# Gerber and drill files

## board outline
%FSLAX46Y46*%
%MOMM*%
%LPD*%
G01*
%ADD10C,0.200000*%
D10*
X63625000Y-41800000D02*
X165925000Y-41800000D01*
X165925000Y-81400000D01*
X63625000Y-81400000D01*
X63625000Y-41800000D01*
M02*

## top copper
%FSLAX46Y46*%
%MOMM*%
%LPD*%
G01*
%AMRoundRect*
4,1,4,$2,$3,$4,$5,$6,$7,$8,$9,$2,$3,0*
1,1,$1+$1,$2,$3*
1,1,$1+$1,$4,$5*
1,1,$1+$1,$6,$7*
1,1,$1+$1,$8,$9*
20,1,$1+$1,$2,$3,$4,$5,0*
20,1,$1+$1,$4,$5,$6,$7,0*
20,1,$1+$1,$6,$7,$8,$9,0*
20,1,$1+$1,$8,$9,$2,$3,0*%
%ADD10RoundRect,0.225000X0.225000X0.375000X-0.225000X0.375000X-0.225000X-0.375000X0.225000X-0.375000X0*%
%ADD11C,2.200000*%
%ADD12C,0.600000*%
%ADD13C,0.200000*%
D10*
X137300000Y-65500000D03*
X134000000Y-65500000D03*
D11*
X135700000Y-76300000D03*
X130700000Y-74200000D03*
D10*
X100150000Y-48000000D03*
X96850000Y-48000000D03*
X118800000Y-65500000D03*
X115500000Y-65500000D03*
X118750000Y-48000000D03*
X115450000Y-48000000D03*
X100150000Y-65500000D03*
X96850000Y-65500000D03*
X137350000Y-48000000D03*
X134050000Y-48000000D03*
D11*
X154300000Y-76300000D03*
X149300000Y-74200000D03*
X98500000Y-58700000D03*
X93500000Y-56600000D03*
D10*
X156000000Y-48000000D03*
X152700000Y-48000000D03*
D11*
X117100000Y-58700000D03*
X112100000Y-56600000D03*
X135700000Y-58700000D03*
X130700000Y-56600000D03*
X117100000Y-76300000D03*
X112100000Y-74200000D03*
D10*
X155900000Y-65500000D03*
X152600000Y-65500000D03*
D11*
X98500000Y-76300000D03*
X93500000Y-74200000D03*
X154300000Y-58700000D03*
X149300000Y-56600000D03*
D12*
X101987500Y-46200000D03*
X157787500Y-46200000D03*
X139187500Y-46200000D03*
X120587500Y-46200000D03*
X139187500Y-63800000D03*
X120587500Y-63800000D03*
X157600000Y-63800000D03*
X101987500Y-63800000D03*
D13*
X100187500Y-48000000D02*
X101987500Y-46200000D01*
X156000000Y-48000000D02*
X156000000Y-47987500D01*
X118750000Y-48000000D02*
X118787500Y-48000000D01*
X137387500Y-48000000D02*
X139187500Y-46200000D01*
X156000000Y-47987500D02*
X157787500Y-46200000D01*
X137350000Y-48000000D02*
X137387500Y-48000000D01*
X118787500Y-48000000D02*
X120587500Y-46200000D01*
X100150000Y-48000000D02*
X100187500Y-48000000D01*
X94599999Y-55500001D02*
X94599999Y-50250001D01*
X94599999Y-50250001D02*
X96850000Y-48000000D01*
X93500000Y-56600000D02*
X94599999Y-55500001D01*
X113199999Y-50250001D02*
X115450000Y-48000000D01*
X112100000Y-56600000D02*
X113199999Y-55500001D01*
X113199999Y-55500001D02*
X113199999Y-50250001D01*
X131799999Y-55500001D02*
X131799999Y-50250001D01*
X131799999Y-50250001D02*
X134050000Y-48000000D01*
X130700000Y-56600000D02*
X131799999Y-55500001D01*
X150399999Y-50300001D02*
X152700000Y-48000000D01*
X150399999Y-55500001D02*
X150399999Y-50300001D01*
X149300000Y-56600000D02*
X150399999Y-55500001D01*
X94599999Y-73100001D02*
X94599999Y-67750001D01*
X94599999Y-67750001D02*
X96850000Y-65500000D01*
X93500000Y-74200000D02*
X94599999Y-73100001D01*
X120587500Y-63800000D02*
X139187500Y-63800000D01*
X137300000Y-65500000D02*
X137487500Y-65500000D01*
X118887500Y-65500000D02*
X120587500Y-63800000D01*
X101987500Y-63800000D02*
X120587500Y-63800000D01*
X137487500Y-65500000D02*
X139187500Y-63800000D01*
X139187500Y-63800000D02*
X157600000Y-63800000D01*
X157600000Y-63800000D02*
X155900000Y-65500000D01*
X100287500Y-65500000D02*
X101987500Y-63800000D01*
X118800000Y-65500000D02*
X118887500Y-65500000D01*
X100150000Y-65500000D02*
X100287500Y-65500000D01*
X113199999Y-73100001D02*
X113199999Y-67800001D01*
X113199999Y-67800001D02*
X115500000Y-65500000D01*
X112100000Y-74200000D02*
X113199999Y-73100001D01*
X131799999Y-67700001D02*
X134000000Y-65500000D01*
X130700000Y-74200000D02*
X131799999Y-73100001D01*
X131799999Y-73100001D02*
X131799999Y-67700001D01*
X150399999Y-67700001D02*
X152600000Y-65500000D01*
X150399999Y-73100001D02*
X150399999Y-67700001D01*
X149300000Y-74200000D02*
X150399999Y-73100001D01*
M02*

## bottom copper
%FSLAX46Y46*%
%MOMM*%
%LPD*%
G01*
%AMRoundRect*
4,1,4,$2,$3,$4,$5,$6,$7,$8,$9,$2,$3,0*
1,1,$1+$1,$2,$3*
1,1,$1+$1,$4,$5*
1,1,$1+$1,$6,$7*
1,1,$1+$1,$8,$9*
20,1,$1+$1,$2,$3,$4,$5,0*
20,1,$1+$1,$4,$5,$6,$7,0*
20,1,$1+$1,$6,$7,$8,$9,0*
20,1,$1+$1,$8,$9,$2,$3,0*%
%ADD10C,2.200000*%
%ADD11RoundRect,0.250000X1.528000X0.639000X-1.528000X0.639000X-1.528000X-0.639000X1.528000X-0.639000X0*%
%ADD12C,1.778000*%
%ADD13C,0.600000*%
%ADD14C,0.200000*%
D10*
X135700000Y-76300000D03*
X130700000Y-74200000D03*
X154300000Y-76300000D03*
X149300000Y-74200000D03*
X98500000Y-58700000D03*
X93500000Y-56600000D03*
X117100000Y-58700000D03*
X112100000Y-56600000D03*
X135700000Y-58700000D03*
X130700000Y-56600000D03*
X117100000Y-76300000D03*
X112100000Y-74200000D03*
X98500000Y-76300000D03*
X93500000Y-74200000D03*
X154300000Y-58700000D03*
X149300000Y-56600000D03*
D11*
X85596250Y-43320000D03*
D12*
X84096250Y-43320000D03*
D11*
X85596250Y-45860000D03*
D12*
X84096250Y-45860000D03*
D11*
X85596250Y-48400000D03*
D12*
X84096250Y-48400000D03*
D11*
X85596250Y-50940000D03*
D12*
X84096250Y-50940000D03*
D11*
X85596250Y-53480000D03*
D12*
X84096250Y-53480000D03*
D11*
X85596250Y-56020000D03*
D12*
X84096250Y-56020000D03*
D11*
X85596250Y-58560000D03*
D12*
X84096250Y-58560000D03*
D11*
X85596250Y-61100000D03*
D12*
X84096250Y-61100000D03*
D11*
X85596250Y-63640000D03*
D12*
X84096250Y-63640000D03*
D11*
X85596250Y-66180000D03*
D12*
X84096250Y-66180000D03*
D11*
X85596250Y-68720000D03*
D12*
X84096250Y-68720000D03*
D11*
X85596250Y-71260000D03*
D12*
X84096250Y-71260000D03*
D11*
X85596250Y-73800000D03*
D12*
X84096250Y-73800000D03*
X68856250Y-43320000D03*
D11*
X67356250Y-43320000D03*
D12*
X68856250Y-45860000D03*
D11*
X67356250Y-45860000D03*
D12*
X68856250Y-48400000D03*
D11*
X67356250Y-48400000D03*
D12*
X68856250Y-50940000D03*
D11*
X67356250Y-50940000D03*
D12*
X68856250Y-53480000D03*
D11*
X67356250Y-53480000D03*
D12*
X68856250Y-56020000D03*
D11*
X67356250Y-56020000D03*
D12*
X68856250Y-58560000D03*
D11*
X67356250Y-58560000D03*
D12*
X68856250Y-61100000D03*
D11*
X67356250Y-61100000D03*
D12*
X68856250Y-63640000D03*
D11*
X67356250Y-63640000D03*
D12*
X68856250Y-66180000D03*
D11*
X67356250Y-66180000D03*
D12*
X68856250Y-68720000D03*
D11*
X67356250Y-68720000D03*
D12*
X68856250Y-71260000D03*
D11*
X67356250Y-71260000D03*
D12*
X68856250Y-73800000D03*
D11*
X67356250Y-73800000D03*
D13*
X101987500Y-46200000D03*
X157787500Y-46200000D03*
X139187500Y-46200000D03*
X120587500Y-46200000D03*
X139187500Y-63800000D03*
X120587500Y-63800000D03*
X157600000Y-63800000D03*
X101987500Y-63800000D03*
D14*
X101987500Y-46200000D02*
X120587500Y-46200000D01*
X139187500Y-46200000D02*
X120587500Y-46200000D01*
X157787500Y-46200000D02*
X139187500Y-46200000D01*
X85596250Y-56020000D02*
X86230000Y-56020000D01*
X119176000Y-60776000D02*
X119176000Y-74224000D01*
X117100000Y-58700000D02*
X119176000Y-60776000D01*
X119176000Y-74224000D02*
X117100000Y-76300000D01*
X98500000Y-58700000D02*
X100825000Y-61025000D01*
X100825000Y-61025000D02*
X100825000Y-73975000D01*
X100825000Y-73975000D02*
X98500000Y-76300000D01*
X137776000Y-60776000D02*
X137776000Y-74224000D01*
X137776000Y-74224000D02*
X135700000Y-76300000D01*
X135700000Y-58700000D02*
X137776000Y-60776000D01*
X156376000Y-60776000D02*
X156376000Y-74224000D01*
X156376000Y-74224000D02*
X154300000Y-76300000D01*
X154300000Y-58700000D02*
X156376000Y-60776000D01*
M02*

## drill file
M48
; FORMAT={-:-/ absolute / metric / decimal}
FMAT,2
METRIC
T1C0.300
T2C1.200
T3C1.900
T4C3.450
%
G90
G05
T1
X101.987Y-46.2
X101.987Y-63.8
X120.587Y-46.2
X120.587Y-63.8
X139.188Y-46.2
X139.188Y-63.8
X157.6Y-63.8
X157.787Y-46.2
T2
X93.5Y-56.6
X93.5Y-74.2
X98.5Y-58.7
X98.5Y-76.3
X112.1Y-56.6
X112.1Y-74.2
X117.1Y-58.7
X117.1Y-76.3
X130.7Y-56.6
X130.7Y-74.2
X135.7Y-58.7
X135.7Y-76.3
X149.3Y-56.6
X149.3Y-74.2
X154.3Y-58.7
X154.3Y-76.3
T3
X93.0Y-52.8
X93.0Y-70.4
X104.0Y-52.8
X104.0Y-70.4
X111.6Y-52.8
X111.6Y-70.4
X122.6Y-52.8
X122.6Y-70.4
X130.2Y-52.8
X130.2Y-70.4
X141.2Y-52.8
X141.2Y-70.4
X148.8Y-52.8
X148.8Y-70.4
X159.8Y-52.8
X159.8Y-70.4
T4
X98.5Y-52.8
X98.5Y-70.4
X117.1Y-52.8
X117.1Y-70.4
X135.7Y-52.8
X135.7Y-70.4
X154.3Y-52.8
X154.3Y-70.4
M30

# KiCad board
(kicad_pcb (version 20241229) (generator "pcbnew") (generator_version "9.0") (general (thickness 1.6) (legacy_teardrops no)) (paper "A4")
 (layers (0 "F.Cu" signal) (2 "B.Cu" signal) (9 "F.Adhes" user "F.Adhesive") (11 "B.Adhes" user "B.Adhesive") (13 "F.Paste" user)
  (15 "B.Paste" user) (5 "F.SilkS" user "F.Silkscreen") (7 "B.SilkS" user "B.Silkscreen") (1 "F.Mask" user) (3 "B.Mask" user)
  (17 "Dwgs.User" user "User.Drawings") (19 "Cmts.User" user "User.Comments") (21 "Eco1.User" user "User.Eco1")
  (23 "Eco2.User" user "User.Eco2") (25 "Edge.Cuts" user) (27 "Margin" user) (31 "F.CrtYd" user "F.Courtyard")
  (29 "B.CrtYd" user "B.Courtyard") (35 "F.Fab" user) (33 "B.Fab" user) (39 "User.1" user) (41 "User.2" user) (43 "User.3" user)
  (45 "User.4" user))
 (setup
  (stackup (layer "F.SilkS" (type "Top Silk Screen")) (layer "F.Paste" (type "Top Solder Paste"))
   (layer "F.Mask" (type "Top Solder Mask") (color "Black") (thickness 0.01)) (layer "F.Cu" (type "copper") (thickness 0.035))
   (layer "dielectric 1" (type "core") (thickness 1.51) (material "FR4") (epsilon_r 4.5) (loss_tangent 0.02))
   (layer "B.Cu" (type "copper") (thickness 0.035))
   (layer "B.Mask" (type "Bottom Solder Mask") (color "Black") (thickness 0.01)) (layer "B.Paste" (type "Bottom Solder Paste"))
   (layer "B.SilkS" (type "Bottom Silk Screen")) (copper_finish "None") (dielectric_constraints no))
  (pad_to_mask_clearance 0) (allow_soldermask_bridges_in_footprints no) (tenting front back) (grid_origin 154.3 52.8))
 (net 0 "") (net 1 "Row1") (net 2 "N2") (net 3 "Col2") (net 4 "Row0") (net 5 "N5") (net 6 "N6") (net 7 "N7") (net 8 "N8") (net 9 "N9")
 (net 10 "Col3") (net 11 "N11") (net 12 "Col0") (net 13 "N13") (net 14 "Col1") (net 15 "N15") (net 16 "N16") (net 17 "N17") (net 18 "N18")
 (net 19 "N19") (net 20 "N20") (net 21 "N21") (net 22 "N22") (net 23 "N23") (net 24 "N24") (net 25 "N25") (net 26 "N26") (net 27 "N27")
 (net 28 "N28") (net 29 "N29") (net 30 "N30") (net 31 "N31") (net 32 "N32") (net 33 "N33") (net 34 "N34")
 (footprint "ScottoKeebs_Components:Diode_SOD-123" (layer "F.Cu") (at 135.65 65.5 180)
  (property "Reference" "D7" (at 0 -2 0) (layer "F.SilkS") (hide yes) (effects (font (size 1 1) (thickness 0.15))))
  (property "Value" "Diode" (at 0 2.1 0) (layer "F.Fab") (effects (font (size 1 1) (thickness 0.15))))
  (pad "1" smd roundrect (at -1.65 0 180) (size 0.9 1.2) (layers "F.Cu" "F.Mask" "F.Paste") (roundrect_rratio 0.25) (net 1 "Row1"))
  (pad "2" smd roundrect (at 1.65 0 180) (size 0.9 1.2) (layers "F.Cu" "F.Mask" "F.Paste") (roundrect_rratio 0.25) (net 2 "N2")))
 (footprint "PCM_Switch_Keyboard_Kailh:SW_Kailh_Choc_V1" (layer "F.Cu") (at 135.7 70.4 180)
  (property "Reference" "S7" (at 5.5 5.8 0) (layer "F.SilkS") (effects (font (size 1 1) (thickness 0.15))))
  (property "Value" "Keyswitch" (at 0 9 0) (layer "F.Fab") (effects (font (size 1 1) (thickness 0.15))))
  (pad "" np_thru_hole circle (at -5.5 0 180) (size 1.9 1.9) (drill 1.9) (layers "*.Cu" "*.Mask"))
  (pad "" np_thru_hole circle (at 0 0 180) (size 3.45 3.45) (drill 3.45) (layers "*.Cu" "*.Mask"))
  (pad "" np_thru_hole circle (at 5.5 0 180) (size 1.9 1.9) (drill 1.9) (layers "*.Cu" "*.Mask"))
  (pad "1" thru_hole circle (at 0 -5.9 180) (size 2.2 2.2) (drill 1.2) (layers "*.Cu" "*.Mask") (remove_unused_layers no) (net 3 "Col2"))
  (pad "2" thru_hole circle (at 5 -3.8 180) (size 2.2 2.2) (drill 1.2) (layers "*.Cu" "*.Mask") (remove_unused_layers no) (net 2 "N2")))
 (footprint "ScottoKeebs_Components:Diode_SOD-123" (layer "F.Cu") (at 98.5 48 180)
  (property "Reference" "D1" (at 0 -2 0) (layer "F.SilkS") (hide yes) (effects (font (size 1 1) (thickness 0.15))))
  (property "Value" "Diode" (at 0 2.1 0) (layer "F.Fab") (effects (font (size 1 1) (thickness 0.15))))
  (pad "1" smd roundrect (at -1.65 0 180) (size 0.9 1.2) (layers "F.Cu" "F.Mask" "F.Paste") (roundrect_rratio 0.25) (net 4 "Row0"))
  (pad "2" smd roundrect (at 1.65 0 180) (size 0.9 1.2) (layers "F.Cu" "F.Mask" "F.Paste") (roundrect_rratio 0.25) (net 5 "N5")))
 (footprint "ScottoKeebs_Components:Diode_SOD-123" (layer "F.Cu") (at 117.15 65.5 180)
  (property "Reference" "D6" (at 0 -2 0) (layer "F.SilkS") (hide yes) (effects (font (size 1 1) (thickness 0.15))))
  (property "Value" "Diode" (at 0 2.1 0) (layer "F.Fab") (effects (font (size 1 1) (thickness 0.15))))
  (pad "1" smd roundrect (at -1.65 0 180) (size 0.9 1.2) (layers "F.Cu" "F.Mask" "F.Paste") (roundrect_rratio 0.25) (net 1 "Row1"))
  (pad "2" smd roundrect (at 1.65 0 180) (size 0.9 1.2) (layers "F.Cu" "F.Mask" "F.Paste") (roundrect_rratio 0.25) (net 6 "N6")))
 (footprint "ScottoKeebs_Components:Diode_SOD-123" (layer "F.Cu") (at 117.1 48 180)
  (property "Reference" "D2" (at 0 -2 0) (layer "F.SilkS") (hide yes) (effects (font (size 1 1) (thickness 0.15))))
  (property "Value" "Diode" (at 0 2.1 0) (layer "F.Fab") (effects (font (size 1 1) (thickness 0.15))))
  (pad "1" smd roundrect (at -1.65 0 180) (size 0.9 1.2) (layers "F.Cu" "F.Mask" "F.Paste") (roundrect_rratio 0.25) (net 4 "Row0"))
  (pad "2" smd roundrect (at 1.65 0 180) (size 0.9 1.2) (layers "F.Cu" "F.Mask" "F.Paste") (roundrect_rratio 0.25) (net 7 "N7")))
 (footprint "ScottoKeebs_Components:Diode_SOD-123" (layer "F.Cu") (at 98.5 65.5 180)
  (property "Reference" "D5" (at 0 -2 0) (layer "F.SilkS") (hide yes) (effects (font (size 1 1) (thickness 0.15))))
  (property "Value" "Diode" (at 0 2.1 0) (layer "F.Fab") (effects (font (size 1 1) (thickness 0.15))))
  (pad "1" smd roundrect (at -1.65 0 180) (size 0.9 1.2) (layers "F.Cu" "F.Mask" "F.Paste") (roundrect_rratio 0.25) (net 1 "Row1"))
  (pad "2" smd roundrect (at 1.65 0 180) (size 0.9 1.2) (layers "F.Cu" "F.Mask" "F.Paste") (roundrect_rratio 0.25) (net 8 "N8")))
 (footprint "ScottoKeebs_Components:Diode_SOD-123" (layer "F.Cu") (at 135.7 48 180)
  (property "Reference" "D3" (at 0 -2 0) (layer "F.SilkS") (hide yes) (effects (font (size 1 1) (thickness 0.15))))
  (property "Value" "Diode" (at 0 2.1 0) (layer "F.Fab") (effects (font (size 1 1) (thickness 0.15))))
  (pad "1" smd roundrect (at -1.65 0 180) (size 0.9 1.2) (layers "F.Cu" "F.Mask" "F.Paste") (roundrect_rratio 0.25) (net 4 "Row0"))
  (pad "2" smd roundrect (at 1.65 0 180) (size 0.9 1.2) (layers "F.Cu" "F.Mask" "F.Paste") (roundrect_rratio 0.25) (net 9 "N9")))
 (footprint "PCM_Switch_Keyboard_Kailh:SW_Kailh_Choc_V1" (layer "F.Cu") (at 154.3 70.4 180)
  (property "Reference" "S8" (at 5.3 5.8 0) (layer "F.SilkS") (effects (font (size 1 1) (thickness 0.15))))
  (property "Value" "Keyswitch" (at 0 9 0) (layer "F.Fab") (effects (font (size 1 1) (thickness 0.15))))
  (pad "" np_thru_hole circle (at -5.5 0 180) (size 1.9 1.9) (drill 1.9) (layers "*.Cu" "*.Mask"))
  (pad "" np_thru_hole circle (at 0 0 180) (size 3.45 3.45) (drill 3.45) (layers "*.Cu" "*.Mask"))
  (pad "" np_thru_hole circle (at 5.5 0 180) (size 1.9 1.9) (drill 1.9) (layers "*.Cu" "*.Mask"))
  (pad "1" thru_hole circle (at 0 -5.9 180) (size 2.2 2.2) (drill 1.2) (layers "*.Cu" "*.Mask") (remove_unused_layers no) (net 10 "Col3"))
  (pad "2" thru_hole circle (at 5 -3.8 180) (size 2.2 2.2) (drill 1.2) (layers "*.Cu" "*.Mask") (remove_unused_layers no) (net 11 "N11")))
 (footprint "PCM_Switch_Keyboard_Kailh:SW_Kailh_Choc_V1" (layer "F.Cu") (at 98.5 52.8 180)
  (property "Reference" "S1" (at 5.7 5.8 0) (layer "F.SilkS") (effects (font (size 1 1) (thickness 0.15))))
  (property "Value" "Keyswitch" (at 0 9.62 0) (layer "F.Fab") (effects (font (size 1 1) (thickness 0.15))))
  (pad "" np_thru_hole circle (at -5.5 0 180) (size 1.9 1.9) (drill 1.9) (layers "*.Cu" "*.Mask"))
  (pad "" np_thru_hole circle (at 0 0 180) (size 3.45 3.45) (drill 3.45) (layers "*.Cu" "*.Mask"))
  (pad "" np_thru_hole circle (at 5.5 0 180) (size 1.9 1.9) (drill 1.9) (layers "*.Cu" "*.Mask"))
  (pad "1" thru_hole circle (at 0 -5.9 180) (size 2.2 2.2) (drill 1.2) (layers "*.Cu" "*.Mask") (remove_unused_layers no) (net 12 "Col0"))
  (pad "2" thru_hole circle (at 5 -3.8 180) (size 2.2 2.2) (drill 1.2) (layers "*.Cu" "*.Mask") (remove_unused_layers no) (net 5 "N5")))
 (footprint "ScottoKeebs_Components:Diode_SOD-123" (layer "F.Cu") (at 154.35 48 180)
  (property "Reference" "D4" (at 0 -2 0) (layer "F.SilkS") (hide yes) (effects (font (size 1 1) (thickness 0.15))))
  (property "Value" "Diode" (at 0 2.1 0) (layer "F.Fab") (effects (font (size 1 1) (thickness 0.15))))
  (pad "1" smd roundrect (at -1.65 0 180) (size 0.9 1.2) (layers "F.Cu" "F.Mask" "F.Paste") (roundrect_rratio 0.25) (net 4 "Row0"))
  (pad "2" smd roundrect (at 1.65 0 180) (size 0.9 1.2) (layers "F.Cu" "F.Mask" "F.Paste") (roundrect_rratio 0.25) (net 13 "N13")))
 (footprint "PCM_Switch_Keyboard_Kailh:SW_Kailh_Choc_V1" (layer "F.Cu") (at 117.1 52.8 180)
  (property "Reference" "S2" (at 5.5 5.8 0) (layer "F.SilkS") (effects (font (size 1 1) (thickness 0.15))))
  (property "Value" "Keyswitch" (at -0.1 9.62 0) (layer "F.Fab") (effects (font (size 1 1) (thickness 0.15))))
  (pad "" np_thru_hole circle (at -5.5 0 180) (size 1.9 1.9) (drill 1.9) (layers "*.Cu" "*.Mask"))
  (pad "" np_thru_hole circle (at 0 0 180) (size 3.45 3.45) (drill 3.45) (layers "*.Cu" "*.Mask"))
  (pad "" np_thru_hole circle (at 5.5 0 180) (size 1.9 1.9) (drill 1.9) (layers "*.Cu" "*.Mask"))
  (pad "1" thru_hole circle (at 0 -5.9 180) (size 2.2 2.2) (drill 1.2) (layers "*.Cu" "*.Mask") (remove_unused_layers no) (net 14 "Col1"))
  (pad "2" thru_hole circle (at 5 -3.8 180) (size 2.2 2.2) (drill 1.2) (layers "*.Cu" "*.Mask") (remove_unused_layers no) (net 7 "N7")))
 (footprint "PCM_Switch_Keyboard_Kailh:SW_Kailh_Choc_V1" (layer "F.Cu") (at 135.7 52.8 180)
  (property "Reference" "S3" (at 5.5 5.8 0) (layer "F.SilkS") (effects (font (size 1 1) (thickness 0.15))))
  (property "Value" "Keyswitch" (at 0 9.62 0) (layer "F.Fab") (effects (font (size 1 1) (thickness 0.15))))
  (pad "" np_thru_hole circle (at -5.5 0 180) (size 1.9 1.9) (drill 1.9) (layers "*.Cu" "*.Mask"))
  (pad "" np_thru_hole circle (at 0 0 180) (size 3.45 3.45) (drill 3.45) (layers "*.Cu" "*.Mask"))
  (pad "" np_thru_hole circle (at 5.5 0 180) (size 1.9 1.9) (drill 1.9) (layers "*.Cu" "*.Mask"))
  (pad "1" thru_hole circle (at 0 -5.9 180) (size 2.2 2.2) (drill 1.2) (layers "*.Cu" "*.Mask") (remove_unused_layers no) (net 3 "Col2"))
  (pad "2" thru_hole circle (at 5 -3.8 180) (size 2.2 2.2) (drill 1.2) (layers "*.Cu" "*.Mask") (remove_unused_layers no) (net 9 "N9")))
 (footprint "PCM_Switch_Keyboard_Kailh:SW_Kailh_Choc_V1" (layer "F.Cu") (at 117.1 70.4 180)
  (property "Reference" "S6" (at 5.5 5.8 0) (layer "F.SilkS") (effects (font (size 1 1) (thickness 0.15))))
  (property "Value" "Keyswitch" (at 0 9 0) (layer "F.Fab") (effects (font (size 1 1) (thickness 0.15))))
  (pad "" np_thru_hole circle (at -5.5 0 180) (size 1.9 1.9) (drill 1.9) (layers "*.Cu" "*.Mask"))
  (pad "" np_thru_hole circle (at 0 0 180) (size 3.45 3.45) (drill 3.45) (layers "*.Cu" "*.Mask"))
  (pad "" np_thru_hole circle (at 5.5 0 180) (size 1.9 1.9) (drill 1.9) (layers "*.Cu" "*.Mask"))
  (pad "1" thru_hole circle (at 0 -5.9 180) (size 2.2 2.2) (drill 1.2) (layers "*.Cu" "*.Mask") (remove_unused_layers no) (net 14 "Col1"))
  (pad "2" thru_hole circle (at 5 -3.8 180) (size 2.2 2.2) (drill 1.2) (layers "*.Cu" "*.Mask") (remove_unused_layers no) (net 6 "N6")))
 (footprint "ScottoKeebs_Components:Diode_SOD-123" (layer "F.Cu") (at 154.25 65.5 180)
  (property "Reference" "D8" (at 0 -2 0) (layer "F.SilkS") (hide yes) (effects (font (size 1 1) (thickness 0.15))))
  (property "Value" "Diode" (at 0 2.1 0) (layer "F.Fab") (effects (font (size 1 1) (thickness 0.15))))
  (pad "1" smd roundrect (at -1.65 0 180) (size 0.9 1.2) (layers "F.Cu" "F.Mask" "F.Paste") (roundrect_rratio 0.25) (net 1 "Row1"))
  (pad "2" smd roundrect (at 1.65 0 180) (size 0.9 1.2) (layers "F.Cu" "F.Mask" "F.Paste") (roundrect_rratio 0.25) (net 11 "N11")))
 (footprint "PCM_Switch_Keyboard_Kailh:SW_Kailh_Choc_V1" (layer "F.Cu") (at 98.5 70.4 180)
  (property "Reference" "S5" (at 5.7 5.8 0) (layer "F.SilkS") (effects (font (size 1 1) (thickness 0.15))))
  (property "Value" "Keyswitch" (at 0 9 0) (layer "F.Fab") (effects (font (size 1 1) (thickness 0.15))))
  (pad "" np_thru_hole circle (at -5.5 0 180) (size 1.9 1.9) (drill 1.9) (layers "*.Cu" "*.Mask"))
  (pad "" np_thru_hole circle (at 0 0 180) (size 3.45 3.45) (drill 3.45) (layers "*.Cu" "*.Mask"))
  (pad "" np_thru_hole circle (at 5.5 0 180) (size 1.9 1.9) (drill 1.9) (layers "*.Cu" "*.Mask"))
  (pad "1" thru_hole circle (at 0 -5.9 180) (size 2.2 2.2) (drill 1.2) (layers "*.Cu" "*.Mask") (remove_unused_layers no) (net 12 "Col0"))
  (pad "2" thru_hole circle (at 5 -3.8 180) (size 2.2 2.2) (drill 1.2) (layers "*.Cu" "*.Mask") (remove_unused_layers no) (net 8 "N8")))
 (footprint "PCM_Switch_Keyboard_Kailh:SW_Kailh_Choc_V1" (layer "F.Cu") (at 154.3 52.8 180)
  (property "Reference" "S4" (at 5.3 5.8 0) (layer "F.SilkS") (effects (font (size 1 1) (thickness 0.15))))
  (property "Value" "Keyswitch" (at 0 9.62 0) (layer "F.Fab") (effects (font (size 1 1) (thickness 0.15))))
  (pad "" np_thru_hole circle (at -5.5 0 180) (size 1.9 1.9) (drill 1.9) (layers "*.Cu" "*.Mask"))
  (pad "" np_thru_hole circle (at 0 0 180) (size 3.45 3.45) (drill 3.45) (layers "*.Cu" "*.Mask"))
  (pad "" np_thru_hole circle (at 5.5 0 180) (size 1.9 1.9) (drill 1.9) (layers "*.Cu" "*.Mask"))
  (pad "1" thru_hole circle (at 0 -5.9 180) (size 2.2 2.2) (drill 1.2) (layers "*.Cu" "*.Mask") (remove_unused_layers no) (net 10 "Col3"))
  (pad "2" thru_hole circle (at 5 -3.8 180) (size 2.2 2.2) (drill 1.2) (layers "*.Cu" "*.Mask") (remove_unused_layers no) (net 13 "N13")))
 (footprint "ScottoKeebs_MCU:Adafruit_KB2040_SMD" (layer "B.Cu") (at 76.48625 58.55 180)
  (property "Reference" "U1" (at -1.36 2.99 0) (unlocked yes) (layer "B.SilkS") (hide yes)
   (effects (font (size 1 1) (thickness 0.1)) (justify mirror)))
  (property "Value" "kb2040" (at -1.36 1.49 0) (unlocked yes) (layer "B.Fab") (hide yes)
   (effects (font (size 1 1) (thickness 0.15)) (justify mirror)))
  (pad "1" smd roundrect (at -9.11 15.23 180) (size 3.556 1.778) (layers "B.Cu" "B.Mask") (roundrect_rratio 0.1406074241) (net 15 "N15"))
  (pad "1" smd circle (at -7.61 15.23 180) (size 1.778 1.778) (layers "B.Cu" "B.Mask" "B.Paste") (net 15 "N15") (solder_mask_margin 0.0508)
   (thermal_bridge_angle 0))
  (pad "2" smd roundrect (at -9.11 12.69 180) (size 3.556 1.778) (layers "B.Cu" "B.Mask") (roundrect_rratio 0.1406074241) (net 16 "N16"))
  (pad "2" smd circle (at -7.61 12.69 180) (size 1.778 1.778) (layers "B.Cu" "B.Mask" "B.Paste") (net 16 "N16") (solder_mask_margin 0.0508)
   (thermal_bridge_angle 0))
  (pad "3" smd roundrect (at -9.11 10.15 180) (size 3.556 1.778) (layers "B.Cu" "B.Mask") (roundrect_rratio 0.1406074241) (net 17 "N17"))
  (pad "3" smd circle (at -7.61 10.15 180) (size 1.778 1.778) (layers "B.Cu" "B.Mask" "B.Paste") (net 17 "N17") (solder_mask_margin 0.0508)
   (thermal_bridge_angle 0))
  (pad "4" smd roundrect (at -9.11 7.61 180) (size 3.556 1.778) (layers "B.Cu" "B.Mask") (roundrect_rratio 0.1406074241) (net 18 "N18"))
  (pad "4" smd circle (at -7.61 7.61 180) (size 1.778 1.778) (layers "B.Cu" "B.Mask" "B.Paste") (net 18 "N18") (solder_mask_margin 0.0508)
   (thermal_bridge_angle 0))
  (pad "5" smd roundrect (at -9.11 5.07 180) (size 3.556 1.778) (layers "B.Cu" "B.Mask") (roundrect_rratio 0.1406074241) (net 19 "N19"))
  (pad "5" smd circle (at -7.61 5.07 180) (size 1.778 1.778) (layers "B.Cu" "B.Mask" "B.Paste") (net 19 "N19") (solder_mask_margin 0.0508)
   (thermal_bridge_angle 0))
  (pad "6" smd roundrect (at -9.11 2.53 180) (size 3.556 1.778) (layers "B.Cu" "B.Mask") (roundrect_rratio 0.1406074241) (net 1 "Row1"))
  (pad "6" smd circle (at -7.61 2.53 180) (size 1.778 1.778) (layers "B.Cu" "B.Mask" "B.Paste") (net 1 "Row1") (solder_mask_margin 0.0508)
   (thermal_bridge_angle 0))
  (pad "7" smd roundrect (at -9.11 -0.01 180) (size 3.556 1.778) (layers "B.Cu" "B.Mask") (roundrect_rratio 0.1406074241) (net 4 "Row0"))
  (pad "7" smd circle (at -7.61 -0.01 180) (size 1.778 1.778) (layers "B.Cu" "B.Mask" "B.Paste") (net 4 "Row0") (solder_mask_margin 0.0508)
   (thermal_bridge_angle 0))
  (pad "8" smd roundrect (at -9.11 -2.55 180) (size 3.556 1.778) (layers "B.Cu" "B.Mask") (roundrect_rratio 0.1406074241) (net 10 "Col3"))
  (pad "8" smd circle (at -7.61 -2.55 180) (size 1.778 1.778) (layers "B.Cu" "B.Mask" "B.Paste") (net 10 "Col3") (solder_mask_margin 0.0508)
   (thermal_bridge_angle 0))
  (pad "9" smd roundrect (at -9.11 -5.09 180) (size 3.556 1.778) (layers "B.Cu" "B.Mask") (roundrect_rratio 0.1406074241) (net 3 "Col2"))
  (pad "9" smd circle (at -7.61 -5.09 180) (size 1.778 1.778) (layers "B.Cu" "B.Mask" "B.Paste") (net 3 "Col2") (solder_mask_margin 0.0508)
   (thermal_bridge_angle 0))
  (pad "10" smd roundrect (at -9.11 -7.63 180) (size 3.556 1.778) (layers "B.Cu" "B.Mask") (roundrect_rratio 0.1406074241) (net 14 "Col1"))
  (pad "10" smd circle (at -7.61 -7.63 180) (size 1.778 1.778) (layers "B.Cu" "B.Mask" "B.Paste") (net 14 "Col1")
   (solder_mask_margin 0.0508) (thermal_bridge_angle 0))
  (pad "11" smd roundrect (at -9.11 -10.17 180) (size 3.556 1.778) (layers "B.Cu" "B.Mask") (roundrect_rratio 0.1406074241) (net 12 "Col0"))
  (pad "11" smd circle (at -7.61 -10.17 180) (size 1.778 1.778) (layers "B.Cu" "B.Mask" "B.Paste") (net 12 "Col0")
   (solder_mask_margin 0.0508) (thermal_bridge_angle 0))
  (pad "12" smd roundrect (at -9.11 -12.71 180) (size 3.556 1.778) (layers "B.Cu" "B.Mask") (roundrect_rratio 0.1406074241) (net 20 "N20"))
  (pad "12" smd circle (at -7.61 -12.71 180) (size 1.778 1.778) (layers "B.Cu" "B.Mask" "B.Paste") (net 20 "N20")
   (solder_mask_margin 0.0508) (thermal_bridge_angle 0))
  (pad "13" smd roundrect (at -9.11 -15.25 180) (size 3.556 1.778) (layers "B.Cu" "B.Mask") (roundrect_rratio 0.1406074241) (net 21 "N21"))
  (pad "13" smd circle (at -7.61 -15.25 180) (size 1.778 1.778) (layers "B.Cu" "B.Mask" "B.Paste") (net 21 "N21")
   (solder_mask_margin 0.0508) (thermal_bridge_angle 0))
  (pad "14" smd circle (at 7.63 15.23 180) (size 1.778 1.778) (layers "B.Cu" "B.Mask" "B.Paste") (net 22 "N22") (solder_mask_margin 0.0508)
   (thermal_bridge_angle 0))
  (pad "14" smd roundrect (at 9.13 15.23 180) (size 3.556 1.778) (layers "B.Cu" "B.Mask") (roundrect_rratio 0.1406074241) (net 22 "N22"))
  (pad "15" smd circle (at 7.63 12.69 180) (size 1.778 1.778) (layers "B.Cu" "B.Mask" "B.Paste") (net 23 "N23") (solder_mask_margin 0.0508)
   (thermal_bridge_angle 0))
  (pad "15" smd roundrect (at 9.13 12.69 180) (size 3.556 1.778) (layers "B.Cu" "B.Mask") (roundrect_rratio 0.1406074241) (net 23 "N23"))
  (pad "16" smd circle (at 7.63 10.15 180) (size 1.778 1.778) (layers "B.Cu" "B.Mask" "B.Paste") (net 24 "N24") (solder_mask_margin 0.0508)
   (thermal_bridge_angle 0))
  (pad "16" smd roundrect (at 9.13 10.15 180) (size 3.556 1.778) (layers "B.Cu" "B.Mask") (roundrect_rratio 0.1406074241) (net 24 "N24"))
  (pad "17" smd circle (at 7.63 7.61 180) (size 1.778 1.778) (layers "B.Cu" "B.Mask" "B.Paste") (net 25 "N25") (solder_mask_margin 0.0508)
   (thermal_bridge_angle 0))
  (pad "17" smd roundrect (at 9.13 7.61 180) (size 3.556 1.778) (layers "B.Cu" "B.Mask") (roundrect_rratio 0.1406074241) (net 25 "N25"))
  (pad "18" smd circle (at 7.63 5.07 180) (size 1.778 1.778) (layers "B.Cu" "B.Mask" "B.Paste") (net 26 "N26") (solder_mask_margin 0.0508)
   (thermal_bridge_angle 0))
  (pad "18" smd roundrect (at 9.13 5.07 180) (size 3.556 1.778) (layers "B.Cu" "B.Mask") (roundrect_rratio 0.1406074241) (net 26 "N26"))
  (pad "19" smd circle (at 7.63 2.53 180) (size 1.778 1.778) (layers "B.Cu" "B.Mask" "B.Paste") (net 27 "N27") (solder_mask_margin 0.0508)
   (thermal_bridge_angle 0))
  (pad "19" smd roundrect (at 9.13 2.53 180) (size 3.556 1.778) (layers "B.Cu" "B.Mask") (roundrect_rratio 0.1406074241) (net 27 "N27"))
  (pad "20" smd circle (at 7.63 -0.01 180) (size 1.778 1.778) (layers "B.Cu" "B.Mask" "B.Paste") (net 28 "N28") (solder_mask_margin 0.0508)
   (thermal_bridge_angle 0))
  (pad "20" smd roundrect (at 9.13 -0.01 180) (size 3.556 1.778) (layers "B.Cu" "B.Mask") (roundrect_rratio 0.1406074241) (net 28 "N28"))
  (pad "21" smd circle (at 7.63 -2.55 180) (size 1.778 1.778) (layers "B.Cu" "B.Mask" "B.Paste") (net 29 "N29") (solder_mask_margin 0.0508)
   (thermal_bridge_angle 0))
  (pad "21" smd roundrect (at 9.13 -2.55 180) (size 3.556 1.778) (layers "B.Cu" "B.Mask") (roundrect_rratio 0.1406074241) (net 29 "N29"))
  (pad "22" smd circle (at 7.63 -5.09 180) (size 1.778 1.778) (layers "B.Cu" "B.Mask" "B.Paste") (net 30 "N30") (solder_mask_margin 0.0508)
   (thermal_bridge_angle 0))
  (pad "22" smd roundrect (at 9.13 -5.09 180) (size 3.556 1.778) (layers "B.Cu" "B.Mask") (roundrect_rratio 0.1406074241) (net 30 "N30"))
  (pad "23" smd circle (at 7.63 -7.63 180) (size 1.778 1.778) (layers "B.Cu" "B.Mask" "B.Paste") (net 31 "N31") (solder_mask_margin 0.0508)
   (thermal_bridge_angle 0))
  (pad "23" smd roundrect (at 9.13 -7.63 180) (size 3.556 1.778) (layers "B.Cu" "B.Mask") (roundrect_rratio 0.1406074241) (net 31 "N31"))
  (pad "24" smd circle (at 7.63 -10.17 180) (size 1.778 1.778) (layers "B.Cu" "B.Mask" "B.Paste") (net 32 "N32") (solder_mask_margin 0.0508)
   (thermal_bridge_angle 0))
  (pad "24" smd roundrect (at 9.13 -10.17 180) (size 3.556 1.778) (layers "B.Cu" "B.Mask") (roundrect_rratio 0.1406074241) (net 32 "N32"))
  (pad "25" smd circle (at 7.63 -12.71 180) (size 1.778 1.778) (layers "B.Cu" "B.Mask" "B.Paste") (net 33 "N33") (solder_mask_margin 0.0508)
   (thermal_bridge_angle 0))
  (pad "25" smd roundrect (at 9.13 -12.71 180) (size 3.556 1.778) (layers "B.Cu" "B.Mask") (roundrect_rratio 0.1406074241) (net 33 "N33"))
  (pad "26" smd circle (at 7.63 -15.25 180) (size 1.778 1.778) (layers "B.Cu" "B.Mask" "B.Paste") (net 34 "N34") (solder_mask_margin 0.0508)
   (thermal_bridge_angle 0))
  (pad "26" smd roundrect (at 9.13 -15.25 180) (size 3.556 1.778) (layers "B.Cu" "B.Mask") (roundrect_rratio 0.1406074241) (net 34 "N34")))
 (gr_rect (start 63.625 41.8) (end 165.925 81.4) (stroke (width 0.2) (type solid)) (fill no) (layer "Edge.Cuts"))
 (segment (start 100.1875 48) (end 101.9875 46.2) (width 0.2) (layer "F.Cu") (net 4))
 (segment (start 156 48) (end 156 47.9875) (width 0.2) (layer "F.Cu") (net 4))
 (segment (start 118.75 48) (end 118.7875 48) (width 0.2) (layer "F.Cu") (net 4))
 (segment (start 137.3875 48) (end 139.1875 46.2) (width 0.2) (layer "F.Cu") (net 4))
 (segment (start 156 47.9875) (end 157.7875 46.2) (width 0.2) (layer "F.Cu") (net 4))
 (segment (start 137.35 48) (end 137.3875 48) (width 0.2) (layer "F.Cu") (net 4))
 (segment (start 118.7875 48) (end 120.5875 46.2) (width 0.2) (layer "F.Cu") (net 4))
 (segment (start 100.15 48) (end 100.1875 48) (width 0.2) (layer "F.Cu") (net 4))
 (via (at 101.9875 46.2) (size 0.6) (drill 0.3) (layers "F.Cu" "B.Cu") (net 4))
 (via (at 157.7875 46.2) (size 0.6) (drill 0.3) (layers "F.Cu" "B.Cu") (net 4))
 (via (at 139.1875 46.2) (size 0.6) (drill 0.3) (layers "F.Cu" "B.Cu") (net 4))
 (via (at 120.5875 46.2) (size 0.6) (drill 0.3) (layers "F.Cu" "B.Cu") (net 4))
 (segment (start 101.9875 46.2) (end 120.5875 46.2) (width 0.2) (layer "B.Cu") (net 4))
 (segment (start 139.1875 46.2) (end 120.5875 46.2) (width 0.2) (layer "B.Cu") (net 4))
 (segment (start 157.7875 46.2) (end 139.1875 46.2) (width 0.2) (layer "B.Cu") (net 4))
 (segment (start 94.599999 55.500001) (end 94.599999 50.250001) (width 0.2) (layer "F.Cu") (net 5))
 (segment (start 94.599999 50.250001) (end 96.85 48) (width 0.2) (layer "F.Cu") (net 5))
 (segment (start 93.5 56.6) (end 94.599999 55.500001) (width 0.2) (layer "F.Cu") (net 5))
 (segment (start 113.199999 50.250001) (end 115.45 48) (width 0.2) (layer "F.Cu") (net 7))
 (segment (start 112.1 56.6) (end 113.199999 55.500001) (width 0.2) (layer "F.Cu") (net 7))
 (segment (start 113.199999 55.500001) (end 113.199999 50.250001) (width 0.2) (layer "F.Cu") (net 7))
 (segment (start 131.799999 55.500001) (end 131.799999 50.250001) (width 0.2) (layer "F.Cu") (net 9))
 (segment (start 131.799999 50.250001) (end 134.05 48) (width 0.2) (layer "F.Cu") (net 9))
 (segment (start 130.7 56.6) (end 131.799999 55.500001) (width 0.2) (layer "F.Cu") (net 9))
 (segment (start 150.399999 50.300001) (end 152.7 48) (width 0.2) (layer "F.Cu") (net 13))
 (segment (start 150.399999 55.500001) (end 150.399999 50.300001) (width 0.2) (layer "F.Cu") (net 13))
 (segment (start 149.3 56.6) (end 150.399999 55.500001) (width 0.2) (layer "F.Cu") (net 13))
 (segment (start 94.599999 73.100001) (end 94.599999 67.750001) (width 0.2) (layer "F.Cu") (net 8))
 (segment (start 94.599999 67.750001) (end 96.85 65.5) (width 0.2) (layer "F.Cu") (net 8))
 (segment (start 93.5 74.2) (end 94.599999 73.100001) (width 0.2) (layer "F.Cu") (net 8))
 (segment (start 120.5875 63.8) (end 139.1875 63.8) (width 0.2) (layer "F.Cu") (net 1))
 (segment (start 137.3 65.5) (end 137.4875 65.5) (width 0.2) (layer "F.Cu") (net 1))
 (segment (start 118.8875 65.5) (end 120.5875 63.8) (width 0.2) (layer "F.Cu") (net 1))
 (segment (start 101.9875 63.8) (end 120.5875 63.8) (width 0.2) (layer "F.Cu") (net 1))
 (segment (start 137.4875 65.5) (end 139.1875 63.8) (width 0.2) (layer "F.Cu") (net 1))
 (segment (start 139.1875 63.8) (end 157.6 63.8) (width 0.2) (layer "F.Cu") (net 1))
 (segment (start 157.6 63.8) (end 155.9 65.5) (width 0.2) (layer "F.Cu") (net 1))
 (segment (start 100.2875 65.5) (end 101.9875 63.8) (width 0.2) (layer "F.Cu") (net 1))
 (segment (start 118.8 65.5) (end 118.8875 65.5) (width 0.2) (layer "F.Cu") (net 1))
 (segment (start 100.15 65.5) (end 100.2875 65.5) (width 0.2) (layer "F.Cu") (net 1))
 (via (at 139.1875 63.8) (size 0.6) (drill 0.3) (layers "F.Cu" "B.Cu") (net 1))
 (via (at 120.5875 63.8) (size 0.6) (drill 0.3) (layers "F.Cu" "B.Cu") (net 1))
 (via (at 157.6 63.8) (size 0.6) (drill 0.3) (layers "F.Cu" "B.Cu") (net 1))
 (via (at 101.9875 63.8) (size 0.6) (drill 0.3) (layers "F.Cu" "B.Cu") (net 1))
 (segment (start 85.59625 56.02) (end 86.23 56.02) (width 0.2) (layer "B.Cu") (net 1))
 (segment (start 113.199999 73.100001) (end 113.199999 67.800001) (width 0.2) (layer "F.Cu") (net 6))
 (segment (start 113.199999 67.800001) (end 115.5 65.5) (width 0.2) (layer "F.Cu") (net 6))
 (segment (start 112.1 74.2) (end 113.199999 73.100001) (width 0.2) (layer "F.Cu") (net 6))
 (segment (start 131.799999 67.700001) (end 134 65.5) (width 0.2) (layer "F.Cu") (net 2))
 (segment (start 130.7 74.2) (end 131.799999 73.100001) (width 0.2) (layer "F.Cu") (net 2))
 (segment (start 131.799999 73.100001) (end 131.799999 67.700001) (width 0.2) (layer "F.Cu") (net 2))
 (segment (start 150.399999 67.700001) (end 152.6 65.5) (width 0.2) (layer "F.Cu") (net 11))
 (segment (start 150.399999 73.100001) (end 150.399999 67.700001) (width 0.2) (layer "F.Cu") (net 11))
 (segment (start 149.3 74.2) (end 150.399999 73.100001) (width 0.2) (layer "F.Cu") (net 11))
 (segment (start 119.176 60.776) (end 119.176 74.224) (width 0.2) (layer "B.Cu") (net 14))
 (segment (start 117.1 58.7) (end 119.176 60.776) (width 0.2) (layer "B.Cu") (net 14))
 (segment (start 119.176 74.224) (end 117.1 76.3) (width 0.2) (layer "B.Cu") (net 14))
 (segment (start 98.5 58.7) (end 100.825 61.025) (width 0.2) (layer "B.Cu") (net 12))
 (segment (start 100.825 61.025) (end 100.825 73.975) (width 0.2) (layer "B.Cu") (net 12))
 (segment (start 100.825 73.975) (end 98.5 76.3) (width 0.2) (layer "B.Cu") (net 12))
 (segment (start 137.776 60.776) (end 137.776 74.224) (width 0.2) (layer "B.Cu") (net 3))
 (segment (start 137.776 74.224) (end 135.7 76.3) (width 0.2) (layer "B.Cu") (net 3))
 (segment (start 135.7 58.7) (end 137.776 60.776) (width 0.2) (layer "B.Cu") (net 3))
 (segment (start 156.376 60.776) (end 156.376 74.224) (width 0.2) (layer "B.Cu") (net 10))
 (segment (start 156.376 74.224) (end 154.3 76.3) (width 0.2) (layer "B.Cu") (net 10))
 (segment (start 154.3 58.7) (end 156.376 60.776) (width 0.2) (layer "B.Cu") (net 10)))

